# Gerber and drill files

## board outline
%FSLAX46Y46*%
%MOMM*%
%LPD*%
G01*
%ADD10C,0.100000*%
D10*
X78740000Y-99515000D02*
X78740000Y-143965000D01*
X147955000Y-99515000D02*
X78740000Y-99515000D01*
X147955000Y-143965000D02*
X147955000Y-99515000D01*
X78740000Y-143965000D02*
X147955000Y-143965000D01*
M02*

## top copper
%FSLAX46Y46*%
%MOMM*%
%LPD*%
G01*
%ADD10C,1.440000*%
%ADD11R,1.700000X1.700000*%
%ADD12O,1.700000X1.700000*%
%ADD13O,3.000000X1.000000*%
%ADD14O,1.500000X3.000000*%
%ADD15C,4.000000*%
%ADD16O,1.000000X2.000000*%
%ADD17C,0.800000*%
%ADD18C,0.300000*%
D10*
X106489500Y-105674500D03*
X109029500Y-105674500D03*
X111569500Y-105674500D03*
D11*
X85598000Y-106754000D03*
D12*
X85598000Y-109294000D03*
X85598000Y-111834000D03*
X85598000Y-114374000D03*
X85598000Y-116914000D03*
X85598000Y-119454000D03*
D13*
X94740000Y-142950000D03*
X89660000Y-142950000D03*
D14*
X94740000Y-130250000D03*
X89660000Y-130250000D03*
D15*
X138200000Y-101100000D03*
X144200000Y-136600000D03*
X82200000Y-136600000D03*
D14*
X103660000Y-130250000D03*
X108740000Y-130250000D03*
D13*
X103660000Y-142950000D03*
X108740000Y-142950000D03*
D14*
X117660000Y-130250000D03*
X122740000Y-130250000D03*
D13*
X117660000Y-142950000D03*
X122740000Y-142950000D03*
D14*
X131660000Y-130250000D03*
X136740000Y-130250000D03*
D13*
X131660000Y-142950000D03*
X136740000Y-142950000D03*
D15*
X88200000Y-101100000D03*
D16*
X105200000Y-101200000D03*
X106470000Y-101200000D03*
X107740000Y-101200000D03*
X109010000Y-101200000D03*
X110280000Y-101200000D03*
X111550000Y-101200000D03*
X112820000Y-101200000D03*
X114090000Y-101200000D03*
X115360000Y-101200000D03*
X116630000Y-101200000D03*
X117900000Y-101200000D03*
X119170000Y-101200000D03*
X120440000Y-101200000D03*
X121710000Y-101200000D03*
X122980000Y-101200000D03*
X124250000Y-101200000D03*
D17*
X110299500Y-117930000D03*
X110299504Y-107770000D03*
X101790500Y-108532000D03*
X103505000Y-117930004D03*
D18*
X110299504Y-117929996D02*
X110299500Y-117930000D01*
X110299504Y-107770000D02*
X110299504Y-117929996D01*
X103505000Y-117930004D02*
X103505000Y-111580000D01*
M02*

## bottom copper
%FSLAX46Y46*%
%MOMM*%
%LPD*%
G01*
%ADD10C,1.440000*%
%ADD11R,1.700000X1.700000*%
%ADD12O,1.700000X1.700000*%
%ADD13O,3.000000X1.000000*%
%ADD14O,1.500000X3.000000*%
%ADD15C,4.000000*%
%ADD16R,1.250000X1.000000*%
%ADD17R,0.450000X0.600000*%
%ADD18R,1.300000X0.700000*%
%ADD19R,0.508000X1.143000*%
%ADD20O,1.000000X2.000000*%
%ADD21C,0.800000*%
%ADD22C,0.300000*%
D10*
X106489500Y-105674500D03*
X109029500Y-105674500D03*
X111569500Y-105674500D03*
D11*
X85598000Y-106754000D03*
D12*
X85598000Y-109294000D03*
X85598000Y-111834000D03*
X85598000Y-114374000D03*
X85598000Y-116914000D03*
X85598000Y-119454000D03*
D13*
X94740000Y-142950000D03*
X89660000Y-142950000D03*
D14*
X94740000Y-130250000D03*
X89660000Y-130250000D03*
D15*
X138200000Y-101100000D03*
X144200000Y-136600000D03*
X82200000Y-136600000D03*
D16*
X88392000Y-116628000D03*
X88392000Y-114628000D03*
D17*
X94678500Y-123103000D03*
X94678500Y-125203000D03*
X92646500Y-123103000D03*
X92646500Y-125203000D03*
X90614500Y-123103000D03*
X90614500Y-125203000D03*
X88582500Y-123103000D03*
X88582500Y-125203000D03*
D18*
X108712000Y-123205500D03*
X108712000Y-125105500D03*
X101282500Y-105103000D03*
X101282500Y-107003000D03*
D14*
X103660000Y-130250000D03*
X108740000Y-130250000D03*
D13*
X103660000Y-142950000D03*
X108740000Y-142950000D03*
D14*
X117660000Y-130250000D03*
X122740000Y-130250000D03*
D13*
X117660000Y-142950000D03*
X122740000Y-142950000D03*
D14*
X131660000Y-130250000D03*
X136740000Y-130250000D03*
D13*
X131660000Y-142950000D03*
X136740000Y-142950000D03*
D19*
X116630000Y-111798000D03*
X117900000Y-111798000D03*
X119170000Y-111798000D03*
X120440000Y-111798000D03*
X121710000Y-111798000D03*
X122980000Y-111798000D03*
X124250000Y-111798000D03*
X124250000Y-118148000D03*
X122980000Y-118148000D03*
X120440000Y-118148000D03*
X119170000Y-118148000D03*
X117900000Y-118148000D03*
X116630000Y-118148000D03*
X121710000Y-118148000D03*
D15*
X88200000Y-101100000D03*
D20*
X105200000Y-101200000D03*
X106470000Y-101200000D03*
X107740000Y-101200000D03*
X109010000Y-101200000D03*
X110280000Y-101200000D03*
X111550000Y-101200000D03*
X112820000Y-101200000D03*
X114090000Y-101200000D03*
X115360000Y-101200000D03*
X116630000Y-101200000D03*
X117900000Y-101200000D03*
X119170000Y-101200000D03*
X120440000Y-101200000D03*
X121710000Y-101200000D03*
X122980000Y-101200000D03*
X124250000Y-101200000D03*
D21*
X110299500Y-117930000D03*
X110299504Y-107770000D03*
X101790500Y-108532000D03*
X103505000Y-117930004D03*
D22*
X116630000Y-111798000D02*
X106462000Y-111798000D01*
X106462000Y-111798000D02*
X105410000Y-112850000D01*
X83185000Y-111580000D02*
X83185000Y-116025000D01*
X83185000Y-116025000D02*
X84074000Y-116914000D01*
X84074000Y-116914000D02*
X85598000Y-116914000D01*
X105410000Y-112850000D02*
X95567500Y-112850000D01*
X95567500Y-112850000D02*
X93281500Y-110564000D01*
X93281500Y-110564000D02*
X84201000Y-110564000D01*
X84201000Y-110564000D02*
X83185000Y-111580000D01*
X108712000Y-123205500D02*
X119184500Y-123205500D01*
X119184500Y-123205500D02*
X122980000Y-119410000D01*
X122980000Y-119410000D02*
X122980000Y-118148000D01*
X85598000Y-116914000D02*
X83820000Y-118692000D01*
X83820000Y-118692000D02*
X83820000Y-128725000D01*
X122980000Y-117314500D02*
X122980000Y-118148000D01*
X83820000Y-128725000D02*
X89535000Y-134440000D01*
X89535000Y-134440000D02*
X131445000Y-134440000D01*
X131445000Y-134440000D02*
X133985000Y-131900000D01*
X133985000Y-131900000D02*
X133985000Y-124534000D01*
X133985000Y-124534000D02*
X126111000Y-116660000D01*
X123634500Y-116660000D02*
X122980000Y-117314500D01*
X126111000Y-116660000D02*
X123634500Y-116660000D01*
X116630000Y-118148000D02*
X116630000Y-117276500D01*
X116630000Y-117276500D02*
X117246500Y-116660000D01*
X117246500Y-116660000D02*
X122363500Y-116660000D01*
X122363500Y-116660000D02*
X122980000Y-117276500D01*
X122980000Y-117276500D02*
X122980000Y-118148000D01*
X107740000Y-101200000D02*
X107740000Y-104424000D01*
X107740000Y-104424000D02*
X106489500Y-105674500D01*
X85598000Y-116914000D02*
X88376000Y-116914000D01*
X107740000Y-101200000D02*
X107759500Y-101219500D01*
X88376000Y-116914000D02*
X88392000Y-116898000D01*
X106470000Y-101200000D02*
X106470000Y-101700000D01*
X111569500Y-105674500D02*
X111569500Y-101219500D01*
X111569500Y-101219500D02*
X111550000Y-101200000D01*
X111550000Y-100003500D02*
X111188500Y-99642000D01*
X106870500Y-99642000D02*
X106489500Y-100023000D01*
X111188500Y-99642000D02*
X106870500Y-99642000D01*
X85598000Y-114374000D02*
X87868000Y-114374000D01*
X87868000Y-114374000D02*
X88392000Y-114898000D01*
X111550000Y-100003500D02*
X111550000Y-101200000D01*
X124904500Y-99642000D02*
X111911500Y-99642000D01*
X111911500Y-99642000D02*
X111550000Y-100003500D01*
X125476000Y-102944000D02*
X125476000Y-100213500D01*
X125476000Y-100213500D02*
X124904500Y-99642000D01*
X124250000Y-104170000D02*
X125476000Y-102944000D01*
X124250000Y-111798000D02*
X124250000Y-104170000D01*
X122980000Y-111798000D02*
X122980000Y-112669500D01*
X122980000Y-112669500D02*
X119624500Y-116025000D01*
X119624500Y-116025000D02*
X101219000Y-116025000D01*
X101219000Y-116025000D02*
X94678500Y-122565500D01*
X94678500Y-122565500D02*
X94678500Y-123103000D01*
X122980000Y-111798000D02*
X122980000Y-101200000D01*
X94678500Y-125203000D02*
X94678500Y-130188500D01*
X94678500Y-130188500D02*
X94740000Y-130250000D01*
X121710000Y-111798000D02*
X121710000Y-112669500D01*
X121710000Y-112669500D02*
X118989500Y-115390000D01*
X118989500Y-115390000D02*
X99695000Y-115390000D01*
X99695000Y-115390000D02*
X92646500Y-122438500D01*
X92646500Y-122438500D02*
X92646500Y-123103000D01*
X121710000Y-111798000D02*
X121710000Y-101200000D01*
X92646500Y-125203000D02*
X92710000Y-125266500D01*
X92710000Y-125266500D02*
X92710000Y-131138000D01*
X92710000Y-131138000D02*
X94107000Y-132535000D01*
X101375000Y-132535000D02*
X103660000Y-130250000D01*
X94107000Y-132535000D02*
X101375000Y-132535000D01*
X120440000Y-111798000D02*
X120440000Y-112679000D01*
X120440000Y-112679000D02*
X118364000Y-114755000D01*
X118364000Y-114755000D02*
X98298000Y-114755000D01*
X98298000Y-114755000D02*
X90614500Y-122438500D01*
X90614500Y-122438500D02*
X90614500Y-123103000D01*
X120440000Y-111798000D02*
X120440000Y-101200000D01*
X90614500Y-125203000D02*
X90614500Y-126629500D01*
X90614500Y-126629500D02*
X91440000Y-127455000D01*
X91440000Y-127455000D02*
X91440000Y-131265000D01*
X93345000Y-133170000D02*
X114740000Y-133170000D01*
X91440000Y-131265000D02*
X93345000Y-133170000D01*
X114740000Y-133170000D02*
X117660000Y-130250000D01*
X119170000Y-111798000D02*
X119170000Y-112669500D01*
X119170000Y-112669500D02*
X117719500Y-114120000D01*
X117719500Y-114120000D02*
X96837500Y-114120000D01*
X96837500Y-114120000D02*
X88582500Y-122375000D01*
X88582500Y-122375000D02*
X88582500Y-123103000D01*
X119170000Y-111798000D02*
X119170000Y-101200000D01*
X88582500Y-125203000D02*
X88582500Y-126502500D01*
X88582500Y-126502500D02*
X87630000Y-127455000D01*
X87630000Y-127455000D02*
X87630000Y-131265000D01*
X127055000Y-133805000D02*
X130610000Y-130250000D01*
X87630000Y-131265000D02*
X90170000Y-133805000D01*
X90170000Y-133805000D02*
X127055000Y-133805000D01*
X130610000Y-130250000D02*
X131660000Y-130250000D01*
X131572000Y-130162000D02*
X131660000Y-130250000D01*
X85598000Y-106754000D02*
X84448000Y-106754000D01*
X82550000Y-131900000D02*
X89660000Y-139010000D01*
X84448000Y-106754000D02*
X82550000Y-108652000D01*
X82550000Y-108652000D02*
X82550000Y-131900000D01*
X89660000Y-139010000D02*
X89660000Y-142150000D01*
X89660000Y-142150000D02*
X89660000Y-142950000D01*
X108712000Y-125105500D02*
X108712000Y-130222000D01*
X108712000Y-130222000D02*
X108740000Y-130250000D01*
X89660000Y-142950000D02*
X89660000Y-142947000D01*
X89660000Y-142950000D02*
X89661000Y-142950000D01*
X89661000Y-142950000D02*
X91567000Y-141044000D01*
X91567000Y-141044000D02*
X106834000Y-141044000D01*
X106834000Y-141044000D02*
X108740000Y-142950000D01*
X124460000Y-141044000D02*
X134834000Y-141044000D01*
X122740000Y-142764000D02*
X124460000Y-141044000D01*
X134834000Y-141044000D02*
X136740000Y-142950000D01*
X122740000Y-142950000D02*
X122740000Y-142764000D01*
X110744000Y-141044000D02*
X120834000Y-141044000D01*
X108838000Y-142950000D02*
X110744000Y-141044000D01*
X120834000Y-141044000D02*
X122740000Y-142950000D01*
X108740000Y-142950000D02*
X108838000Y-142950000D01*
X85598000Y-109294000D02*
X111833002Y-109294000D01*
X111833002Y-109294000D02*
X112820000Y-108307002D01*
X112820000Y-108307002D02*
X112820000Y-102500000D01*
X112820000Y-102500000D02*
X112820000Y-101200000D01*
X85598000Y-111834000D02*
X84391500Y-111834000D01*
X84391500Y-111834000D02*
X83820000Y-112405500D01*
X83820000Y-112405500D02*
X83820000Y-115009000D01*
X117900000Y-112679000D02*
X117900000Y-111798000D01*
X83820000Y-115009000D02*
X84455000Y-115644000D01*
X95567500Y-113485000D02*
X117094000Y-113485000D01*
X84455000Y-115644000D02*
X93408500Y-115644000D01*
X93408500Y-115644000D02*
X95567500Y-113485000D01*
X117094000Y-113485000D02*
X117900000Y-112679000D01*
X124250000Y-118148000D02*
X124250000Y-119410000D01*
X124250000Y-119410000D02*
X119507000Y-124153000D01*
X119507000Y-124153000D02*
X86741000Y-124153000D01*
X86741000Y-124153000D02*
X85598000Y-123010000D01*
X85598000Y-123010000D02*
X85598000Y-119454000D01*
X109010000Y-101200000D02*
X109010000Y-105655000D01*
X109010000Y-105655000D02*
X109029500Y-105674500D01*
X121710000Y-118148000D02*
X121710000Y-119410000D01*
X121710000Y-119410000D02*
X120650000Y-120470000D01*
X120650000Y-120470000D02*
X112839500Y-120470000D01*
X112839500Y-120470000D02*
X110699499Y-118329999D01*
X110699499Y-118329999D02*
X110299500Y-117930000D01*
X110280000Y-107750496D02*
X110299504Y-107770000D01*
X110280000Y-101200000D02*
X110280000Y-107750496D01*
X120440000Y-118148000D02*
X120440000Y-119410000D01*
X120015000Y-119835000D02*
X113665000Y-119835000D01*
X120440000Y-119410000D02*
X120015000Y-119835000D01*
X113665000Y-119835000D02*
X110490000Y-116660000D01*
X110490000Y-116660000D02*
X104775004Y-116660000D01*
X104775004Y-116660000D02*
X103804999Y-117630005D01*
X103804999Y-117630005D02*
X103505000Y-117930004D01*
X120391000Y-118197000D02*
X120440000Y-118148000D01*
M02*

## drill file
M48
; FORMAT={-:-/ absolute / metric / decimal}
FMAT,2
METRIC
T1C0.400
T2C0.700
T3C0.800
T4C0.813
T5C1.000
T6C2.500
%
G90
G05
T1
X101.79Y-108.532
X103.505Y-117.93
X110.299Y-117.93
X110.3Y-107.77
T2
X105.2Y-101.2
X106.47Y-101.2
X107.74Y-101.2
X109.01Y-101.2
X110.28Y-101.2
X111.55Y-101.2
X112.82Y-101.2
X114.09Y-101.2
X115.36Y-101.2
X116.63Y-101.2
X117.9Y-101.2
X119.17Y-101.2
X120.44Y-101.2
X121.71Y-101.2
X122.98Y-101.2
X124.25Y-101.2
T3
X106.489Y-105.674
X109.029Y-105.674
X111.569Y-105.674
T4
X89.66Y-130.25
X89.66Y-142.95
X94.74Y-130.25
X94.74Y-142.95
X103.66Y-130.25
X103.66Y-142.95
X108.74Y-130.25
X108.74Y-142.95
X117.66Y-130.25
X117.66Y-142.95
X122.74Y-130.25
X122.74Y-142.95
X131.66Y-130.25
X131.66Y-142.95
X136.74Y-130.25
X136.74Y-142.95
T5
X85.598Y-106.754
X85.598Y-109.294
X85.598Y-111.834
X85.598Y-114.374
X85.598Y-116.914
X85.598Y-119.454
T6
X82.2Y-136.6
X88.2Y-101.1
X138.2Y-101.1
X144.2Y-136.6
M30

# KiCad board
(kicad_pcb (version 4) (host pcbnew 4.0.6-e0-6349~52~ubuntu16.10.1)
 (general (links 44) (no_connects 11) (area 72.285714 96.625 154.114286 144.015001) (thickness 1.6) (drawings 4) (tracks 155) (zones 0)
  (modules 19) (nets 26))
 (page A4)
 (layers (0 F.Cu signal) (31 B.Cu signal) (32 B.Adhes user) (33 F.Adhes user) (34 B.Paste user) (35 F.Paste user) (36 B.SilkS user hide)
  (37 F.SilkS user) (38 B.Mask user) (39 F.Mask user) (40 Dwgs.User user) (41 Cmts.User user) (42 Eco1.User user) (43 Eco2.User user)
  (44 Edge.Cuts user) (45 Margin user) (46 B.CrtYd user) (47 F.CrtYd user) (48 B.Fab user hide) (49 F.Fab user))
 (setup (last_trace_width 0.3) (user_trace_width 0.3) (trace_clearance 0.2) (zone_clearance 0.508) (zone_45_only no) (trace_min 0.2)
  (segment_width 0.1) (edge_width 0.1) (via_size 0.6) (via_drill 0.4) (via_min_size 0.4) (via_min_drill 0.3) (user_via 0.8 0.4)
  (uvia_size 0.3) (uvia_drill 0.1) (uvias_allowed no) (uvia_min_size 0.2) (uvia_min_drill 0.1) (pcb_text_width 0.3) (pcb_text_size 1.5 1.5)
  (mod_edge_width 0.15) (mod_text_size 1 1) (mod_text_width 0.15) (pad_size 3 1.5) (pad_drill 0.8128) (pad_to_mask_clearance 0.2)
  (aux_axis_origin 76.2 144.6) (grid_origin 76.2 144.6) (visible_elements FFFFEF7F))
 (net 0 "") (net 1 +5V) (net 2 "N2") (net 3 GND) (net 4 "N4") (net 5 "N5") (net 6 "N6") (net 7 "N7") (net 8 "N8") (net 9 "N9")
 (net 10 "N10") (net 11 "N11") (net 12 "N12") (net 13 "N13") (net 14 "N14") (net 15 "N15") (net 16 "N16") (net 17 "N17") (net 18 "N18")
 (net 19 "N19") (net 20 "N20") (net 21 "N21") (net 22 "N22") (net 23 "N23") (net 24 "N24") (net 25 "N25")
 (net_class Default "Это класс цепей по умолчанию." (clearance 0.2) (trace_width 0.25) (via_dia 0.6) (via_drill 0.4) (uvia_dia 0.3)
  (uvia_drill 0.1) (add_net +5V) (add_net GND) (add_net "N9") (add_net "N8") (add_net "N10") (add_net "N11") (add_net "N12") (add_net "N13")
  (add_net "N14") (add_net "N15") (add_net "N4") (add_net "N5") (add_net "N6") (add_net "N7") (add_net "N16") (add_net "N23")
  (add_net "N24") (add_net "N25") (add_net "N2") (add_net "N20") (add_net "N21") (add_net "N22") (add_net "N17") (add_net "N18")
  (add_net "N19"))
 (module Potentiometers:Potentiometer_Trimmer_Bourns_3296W (layer B.Cu) (at 106.4895 105.6745 180)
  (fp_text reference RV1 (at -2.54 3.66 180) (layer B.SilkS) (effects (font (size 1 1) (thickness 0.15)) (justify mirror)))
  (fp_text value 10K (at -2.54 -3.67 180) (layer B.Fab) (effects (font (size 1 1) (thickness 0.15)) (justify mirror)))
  (pad 1 thru_hole circle (at 0 0 180) (size 1.44 1.44) (drill 0.8) (layers *.Cu *.Mask) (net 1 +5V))
  (pad 2 thru_hole circle (at -2.54 0 180) (size 1.44 1.44) (drill 0.8) (layers *.Cu *.Mask) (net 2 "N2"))
  (pad 3 thru_hole circle (at -5.08 0 180) (size 1.44 1.44) (drill 0.8) (layers *.Cu *.Mask) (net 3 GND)))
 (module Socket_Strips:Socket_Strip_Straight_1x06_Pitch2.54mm (layer B.Cu) (at 85.598 106.754 180)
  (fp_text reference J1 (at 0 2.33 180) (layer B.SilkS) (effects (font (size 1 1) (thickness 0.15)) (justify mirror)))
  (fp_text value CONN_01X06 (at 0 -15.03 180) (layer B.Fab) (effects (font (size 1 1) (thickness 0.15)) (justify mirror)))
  (pad 1 thru_hole rect (at 0 0 180) (size 1.7 1.7) (drill 1) (layers *.Cu *.Mask) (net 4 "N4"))
  (pad 2 thru_hole oval (at 0 -2.54 180) (size 1.7 1.7) (drill 1) (layers *.Cu *.Mask) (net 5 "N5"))
  (pad 3 thru_hole oval (at 0 -5.08 180) (size 1.7 1.7) (drill 1) (layers *.Cu *.Mask) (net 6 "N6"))
  (pad 4 thru_hole oval (at 0 -7.62 180) (size 1.7 1.7) (drill 1) (layers *.Cu *.Mask) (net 3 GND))
  (pad 5 thru_hole oval (at 0 -10.16 180) (size 1.7 1.7) (drill 1) (layers *.Cu *.Mask) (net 1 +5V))
  (pad 6 thru_hole oval (at 0 -12.7 180) (size 1.7 1.7) (drill 1) (layers *.Cu *.Mask) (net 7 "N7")))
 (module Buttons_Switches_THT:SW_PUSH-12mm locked (layer F.Cu) (at 92.2 136.6 270)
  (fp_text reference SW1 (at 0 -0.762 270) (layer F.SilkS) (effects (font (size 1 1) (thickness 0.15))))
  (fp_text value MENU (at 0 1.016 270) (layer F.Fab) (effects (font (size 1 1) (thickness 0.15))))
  (pad 1 thru_hole oval (at 6.35 -2.54) (size 3 1) (drill 0.8128) (layers *.Cu *.Mask) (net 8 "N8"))
  (pad 2 thru_hole oval (at 6.35 2.54) (size 3 1) (drill 0.8128) (layers *.Cu *.Mask) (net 4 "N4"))
  (pad 1 thru_hole oval (at -6.35 -2.54 270) (size 3 1.5) (drill 0.8128) (layers *.Cu *.Mask) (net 8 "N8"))
  (pad 2 thru_hole oval (at -6.35 2.54 270) (size 3 1.5) (drill 0.8128) (layers *.Cu *.Mask) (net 4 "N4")))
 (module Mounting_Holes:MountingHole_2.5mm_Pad (layer F.Cu) (at 138.2 101.1)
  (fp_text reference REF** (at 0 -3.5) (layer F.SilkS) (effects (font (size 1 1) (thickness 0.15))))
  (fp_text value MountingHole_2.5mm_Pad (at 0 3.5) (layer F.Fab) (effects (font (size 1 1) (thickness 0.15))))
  (pad 1 thru_hole circle (at 0 0) (size 4 4) (drill 2.5) (layers *.Cu *.Mask)))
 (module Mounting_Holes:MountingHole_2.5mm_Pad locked (layer F.Cu) (at 144.2 136.6)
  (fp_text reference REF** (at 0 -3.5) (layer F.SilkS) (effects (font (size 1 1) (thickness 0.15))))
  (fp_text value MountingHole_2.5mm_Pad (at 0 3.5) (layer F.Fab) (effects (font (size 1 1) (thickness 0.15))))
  (pad 1 thru_hole circle (at 0 0) (size 4 4) (drill 2.5) (layers *.Cu *.Mask)))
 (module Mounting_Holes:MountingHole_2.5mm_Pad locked (layer F.Cu) (at 82.2 136.6)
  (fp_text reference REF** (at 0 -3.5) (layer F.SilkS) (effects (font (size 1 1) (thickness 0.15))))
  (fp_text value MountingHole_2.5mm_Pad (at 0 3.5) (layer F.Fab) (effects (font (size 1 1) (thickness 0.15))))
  (pad 1 thru_hole circle (at 0 0) (size 4 4) (drill 2.5) (layers *.Cu *.Mask)))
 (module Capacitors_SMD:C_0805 (layer B.Cu) (at 88.392 115.628 90)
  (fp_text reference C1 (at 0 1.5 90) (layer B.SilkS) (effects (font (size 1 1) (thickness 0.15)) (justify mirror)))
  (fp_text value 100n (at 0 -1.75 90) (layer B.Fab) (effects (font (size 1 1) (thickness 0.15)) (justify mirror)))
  (pad 1 smd rect (at -1 0 90) (size 1 1.25) (layers B.Cu B.Paste B.Mask) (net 1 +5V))
  (pad 2 smd rect (at 1 0 90) (size 1 1.25) (layers B.Cu B.Paste B.Mask) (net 3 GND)))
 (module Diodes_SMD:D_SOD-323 (layer B.Cu) (at 94.6785 124.153 270)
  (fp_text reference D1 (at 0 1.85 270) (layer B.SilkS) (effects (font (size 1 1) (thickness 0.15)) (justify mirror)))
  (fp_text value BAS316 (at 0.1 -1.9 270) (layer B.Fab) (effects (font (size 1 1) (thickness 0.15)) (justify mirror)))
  (pad 1 smd rect (at -1.05 0 270) (size 0.6 0.45) (layers B.Cu B.Paste B.Mask) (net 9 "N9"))
  (pad 2 smd rect (at 1.05 0 270) (size 0.6 0.45) (layers B.Cu B.Paste B.Mask) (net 8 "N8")))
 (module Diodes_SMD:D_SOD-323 (layer B.Cu) (at 92.6465 124.153 270)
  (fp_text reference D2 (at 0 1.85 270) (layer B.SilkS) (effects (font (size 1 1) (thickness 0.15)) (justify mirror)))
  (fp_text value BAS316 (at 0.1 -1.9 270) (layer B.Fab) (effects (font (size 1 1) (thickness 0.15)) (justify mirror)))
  (pad 1 smd rect (at -1.05 0 270) (size 0.6 0.45) (layers B.Cu B.Paste B.Mask) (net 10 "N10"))
  (pad 2 smd rect (at 1.05 0 270) (size 0.6 0.45) (layers B.Cu B.Paste B.Mask) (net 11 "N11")))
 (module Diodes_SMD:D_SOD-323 (layer B.Cu) (at 90.6145 124.153 270)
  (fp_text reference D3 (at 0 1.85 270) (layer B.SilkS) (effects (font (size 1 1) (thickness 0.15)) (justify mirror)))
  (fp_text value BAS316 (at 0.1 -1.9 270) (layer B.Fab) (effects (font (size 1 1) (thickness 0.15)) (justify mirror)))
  (pad 1 smd rect (at -1.05 0 270) (size 0.6 0.45) (layers B.Cu B.Paste B.Mask) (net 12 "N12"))
  (pad 2 smd rect (at 1.05 0 270) (size 0.6 0.45) (layers B.Cu B.Paste B.Mask) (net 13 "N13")))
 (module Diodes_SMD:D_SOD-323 (layer B.Cu) (at 88.5825 124.153 270)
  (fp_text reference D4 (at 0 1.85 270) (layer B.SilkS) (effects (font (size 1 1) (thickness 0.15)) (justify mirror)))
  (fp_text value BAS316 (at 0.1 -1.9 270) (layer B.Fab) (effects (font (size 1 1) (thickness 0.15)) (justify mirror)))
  (pad 1 smd rect (at -1.05 0 270) (size 0.6 0.45) (layers B.Cu B.Paste B.Mask) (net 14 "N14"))
  (pad 2 smd rect (at 1.05 0 270) (size 0.6 0.45) (layers B.Cu B.Paste B.Mask) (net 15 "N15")))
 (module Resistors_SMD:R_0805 (layer B.Cu) (at 108.712 124.1555 270)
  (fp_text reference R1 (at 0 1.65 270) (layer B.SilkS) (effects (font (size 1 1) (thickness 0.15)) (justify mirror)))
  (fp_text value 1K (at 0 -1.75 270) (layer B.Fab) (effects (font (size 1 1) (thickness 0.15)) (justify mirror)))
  (pad 1 smd rect (at -0.95 0 270) (size 0.7 1.3) (layers B.Cu B.Paste B.Mask) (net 1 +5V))
  (pad 2 smd rect (at 0.95 0 270) (size 0.7 1.3) (layers B.Cu B.Paste B.Mask) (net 4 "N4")))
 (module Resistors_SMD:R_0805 (layer B.Cu) (at 101.2825 106.053 270)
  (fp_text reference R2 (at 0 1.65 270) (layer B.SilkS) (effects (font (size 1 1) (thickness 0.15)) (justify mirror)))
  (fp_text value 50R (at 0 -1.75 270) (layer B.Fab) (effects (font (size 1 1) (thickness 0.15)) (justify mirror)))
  (pad 1 smd rect (at -0.95 0 270) (size 0.7 1.3) (layers B.Cu B.Paste B.Mask) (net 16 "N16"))
  (pad 2 smd rect (at 0.95 0 270) (size 0.7 1.3) (layers B.Cu B.Paste B.Mask) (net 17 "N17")))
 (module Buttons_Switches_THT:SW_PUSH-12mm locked (layer F.Cu) (at 106.2 136.6 90)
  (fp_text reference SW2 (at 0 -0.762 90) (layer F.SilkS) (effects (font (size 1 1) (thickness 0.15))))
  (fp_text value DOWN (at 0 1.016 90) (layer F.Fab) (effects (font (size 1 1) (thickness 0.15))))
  (pad 1 thru_hole oval (at 6.35 -2.54 90) (size 3 1.5) (drill 0.8128) (layers *.Cu *.Mask) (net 11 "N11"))
  (pad 2 thru_hole oval (at 6.35 2.54 90) (size 3 1.5) (drill 0.8128) (layers *.Cu *.Mask) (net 4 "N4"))
  (pad 1 thru_hole oval (at -6.35 -2.54 180) (size 3 1) (drill 0.8128) (layers *.Cu *.Mask) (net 11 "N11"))
  (pad 2 thru_hole oval (at -6.35 2.54 180) (size 3 1) (drill 0.8128) (layers *.Cu *.Mask) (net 4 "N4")))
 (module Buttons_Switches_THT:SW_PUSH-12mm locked (layer F.Cu) (at 120.2 136.6 90)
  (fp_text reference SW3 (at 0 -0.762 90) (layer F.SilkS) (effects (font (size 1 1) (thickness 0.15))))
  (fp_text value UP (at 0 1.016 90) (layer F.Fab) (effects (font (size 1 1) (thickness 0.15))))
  (pad 1 thru_hole oval (at 6.35 -2.54 90) (size 3 1.5) (drill 0.8128) (layers *.Cu *.Mask) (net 13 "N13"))
  (pad 2 thru_hole oval (at 6.35 2.54 90) (size 3 1.5) (drill 0.8128) (layers *.Cu *.Mask) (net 4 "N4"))
  (pad 1 thru_hole oval (at -6.35 -2.54 180) (size 3 1) (drill 0.8128) (layers *.Cu *.Mask) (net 13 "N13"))
  (pad 2 thru_hole oval (at -6.35 2.54 180) (size 3 1) (drill 0.8128) (layers *.Cu *.Mask) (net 4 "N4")))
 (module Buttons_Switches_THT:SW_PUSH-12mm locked (layer F.Cu) (at 134.2 136.6 90)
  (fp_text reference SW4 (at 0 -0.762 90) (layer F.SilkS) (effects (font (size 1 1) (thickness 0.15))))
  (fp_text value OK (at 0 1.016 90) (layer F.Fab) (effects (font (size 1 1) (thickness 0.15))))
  (pad 1 thru_hole oval (at 6.35 -2.54 90) (size 3 1.5) (drill 0.8128) (layers *.Cu *.Mask) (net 15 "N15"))
  (pad 2 thru_hole oval (at 6.35 2.54 90) (size 3 1.5) (drill 0.8128) (layers *.Cu *.Mask) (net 4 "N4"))
  (pad 1 thru_hole oval (at -6.35 -2.54 180) (size 3 1) (drill 0.8128) (layers *.Cu *.Mask) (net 15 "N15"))
  (pad 2 thru_hole oval (at -6.35 2.54 180) (size 3 1) (drill 0.8128) (layers *.Cu *.Mask) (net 4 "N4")))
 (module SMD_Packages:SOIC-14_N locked (layer B.Cu) (at 120.44 115.1)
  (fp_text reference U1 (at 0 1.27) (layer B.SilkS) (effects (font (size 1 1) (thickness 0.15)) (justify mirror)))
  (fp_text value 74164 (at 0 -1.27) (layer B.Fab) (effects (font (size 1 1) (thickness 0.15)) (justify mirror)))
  (pad 1 smd rect (at -3.81 -3.302) (size 0.508 1.143) (layers B.Cu B.Paste B.Mask) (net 1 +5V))
  (pad 2 smd rect (at -2.54 -3.302) (size 0.508 1.143) (layers B.Cu B.Paste B.Mask) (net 6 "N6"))
  (pad 3 smd rect (at -1.27 -3.302) (size 0.508 1.143) (layers B.Cu B.Paste B.Mask) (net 14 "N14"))
  (pad 4 smd rect (at 0 -3.302) (size 0.508 1.143) (layers B.Cu B.Paste B.Mask) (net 12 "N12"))
  (pad 5 smd rect (at 1.27 -3.302) (size 0.508 1.143) (layers B.Cu B.Paste B.Mask) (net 10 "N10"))
  (pad 6 smd rect (at 2.54 -3.302) (size 0.508 1.143) (layers B.Cu B.Paste B.Mask) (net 9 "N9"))
  (pad 7 smd rect (at 3.81 -3.302) (size 0.508 1.143) (layers B.Cu B.Paste B.Mask) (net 3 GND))
  (pad 8 smd rect (at 3.81 3.048) (size 0.508 1.143) (layers B.Cu B.Paste B.Mask) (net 7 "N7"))
  (pad 9 smd rect (at 2.54 3.048) (size 0.508 1.143) (layers B.Cu B.Paste B.Mask) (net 1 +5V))
  (pad 11 smd rect (at 0 3.048) (size 0.508 1.143) (layers B.Cu B.Paste B.Mask) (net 17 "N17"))
  (pad 12 smd rect (at -1.27 3.048) (size 0.508 1.143) (layers B.Cu B.Paste B.Mask) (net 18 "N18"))
  (pad 13 smd rect (at -2.54 3.048) (size 0.508 1.143) (layers B.Cu B.Paste B.Mask) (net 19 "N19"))
  (pad 14 smd rect (at -3.81 3.048) (size 0.508 1.143) (layers B.Cu B.Paste B.Mask) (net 1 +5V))
  (pad 10 smd rect (at 1.27 3.048) (size 0.508 1.143) (layers B.Cu B.Paste B.Mask) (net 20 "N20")))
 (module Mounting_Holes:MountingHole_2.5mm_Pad (layer F.Cu) (at 88.2 101.1)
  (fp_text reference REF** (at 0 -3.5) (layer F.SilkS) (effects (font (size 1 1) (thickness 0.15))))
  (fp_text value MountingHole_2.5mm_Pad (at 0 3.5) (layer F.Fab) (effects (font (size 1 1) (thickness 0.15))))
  (pad 1 thru_hole circle (at 0 0) (size 4 4) (drill 2.5) (layers *.Cu *.Mask)))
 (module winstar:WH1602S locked (layer F.Cu) (at 113.2 115.1)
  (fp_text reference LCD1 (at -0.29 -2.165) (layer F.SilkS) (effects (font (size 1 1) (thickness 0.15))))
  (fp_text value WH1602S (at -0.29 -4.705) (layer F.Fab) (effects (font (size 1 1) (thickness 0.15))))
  (pad 1 thru_hole oval (at -8 -13.9) (size 1 2) (drill 0.7) (layers *.Cu *.Mask) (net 16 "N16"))
  (pad 2 thru_hole oval (at -6.73 -13.9) (size 1 2) (drill 0.7) (layers *.Cu *.Mask) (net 3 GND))
  (pad 3 thru_hole oval (at -5.46 -13.9) (size 1 2) (drill 0.7) (layers *.Cu *.Mask) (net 1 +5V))
  (pad 4 thru_hole oval (at -4.19 -13.9) (size 1 2) (drill 0.7) (layers *.Cu *.Mask) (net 2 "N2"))
  (pad 5 thru_hole oval (at -2.92 -13.9) (size 1 2) (drill 0.7) (layers *.Cu *.Mask) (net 20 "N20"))
  (pad 6 thru_hole oval (at -1.65 -13.9) (size 1 2) (drill 0.7) (layers *.Cu *.Mask) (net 3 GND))
  (pad 7 thru_hole oval (at -0.38 -13.9) (size 1 2) (drill 0.7) (layers *.Cu *.Mask) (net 5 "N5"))
  (pad 8 thru_hole oval (at 0.89 -13.9) (size 1 2) (drill 0.7) (layers *.Cu *.Mask) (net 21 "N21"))
  (pad 9 thru_hole oval (at 2.16 -13.9) (size 1 2) (drill 0.7) (layers *.Cu *.Mask) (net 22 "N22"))
  (pad 10 thru_hole oval (at 3.43 -13.9) (size 1 2) (drill 0.7) (layers *.Cu *.Mask) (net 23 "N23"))
  (pad 11 thru_hole oval (at 4.7 -13.9) (size 1 2) (drill 0.7) (layers *.Cu *.Mask) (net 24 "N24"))
  (pad 12 thru_hole oval (at 5.97 -13.9) (size 1 2) (drill 0.7) (layers *.Cu *.Mask) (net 14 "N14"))
  (pad 13 thru_hole oval (at 7.24 -13.9) (size 1 2) (drill 0.7) (layers *.Cu *.Mask) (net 12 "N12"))
  (pad 14 thru_hole oval (at 8.51 -13.9) (size 1 2) (drill 0.7) (layers *.Cu *.Mask) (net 10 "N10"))
  (pad 15 thru_hole oval (at 9.78 -13.9) (size 1 2) (drill 0.7) (layers *.Cu *.Mask) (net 9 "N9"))
  (pad 16 thru_hole oval (at 11.05 -13.9) (size 1 2) (drill 0.7) (layers *.Cu *.Mask) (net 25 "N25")))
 (gr_line (start 78.74 99.515) (end 78.74 143.965) (layer Edge.Cuts) (width 0.1))
 (gr_line (start 147.955 99.515) (end 78.74 99.515) (layer Edge.Cuts) (width 0.1))
 (gr_line (start 147.955 143.965) (end 147.955 99.515) (layer Edge.Cuts) (width 0.1))
 (gr_line (start 78.74 143.965) (end 147.955 143.965) (layer Edge.Cuts) (width 0.1))
 (segment (start 116.63 111.798) (end 106.462 111.798) (width 0.3) (layer B.Cu) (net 1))
 (segment (start 106.462 111.798) (end 105.41 112.85) (width 0.3) (layer B.Cu) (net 1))
 (segment (start 83.185 111.58) (end 83.185 116.025) (width 0.3) (layer B.Cu) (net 1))
 (segment (start 83.185 116.025) (end 84.074 116.914) (width 0.3) (layer B.Cu) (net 1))
 (segment (start 84.074 116.914) (end 85.598 116.914) (width 0.3) (layer B.Cu) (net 1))
 (segment (start 105.41 112.85) (end 95.5675 112.85) (width 0.3) (layer B.Cu) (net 1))
 (segment (start 95.5675 112.85) (end 93.2815 110.564) (width 0.3) (layer B.Cu) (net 1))
 (segment (start 93.2815 110.564) (end 84.201 110.564) (width 0.3) (layer B.Cu) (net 1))
 (segment (start 84.201 110.564) (end 83.185 111.58) (width 0.3) (layer B.Cu) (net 1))
 (segment (start 108.712 123.2055) (end 119.1845 123.2055) (width 0.3) (layer B.Cu) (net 1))
 (segment (start 119.1845 123.2055) (end 122.98 119.41) (width 0.3) (layer B.Cu) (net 1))
 (segment (start 122.98 119.41) (end 122.98 118.148) (width 0.3) (layer B.Cu) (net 1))
 (segment (start 85.598 116.914) (end 83.82 118.692) (width 0.3) (layer B.Cu) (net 1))
 (segment (start 83.82 118.692) (end 83.82 128.725) (width 0.3) (layer B.Cu) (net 1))
 (segment (start 122.98 117.3145) (end 122.98 118.148) (width 0.3) (layer B.Cu) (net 1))
 (segment (start 83.82 128.725) (end 89.535 134.44) (width 0.3) (layer B.Cu) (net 1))
 (segment (start 89.535 134.44) (end 131.445 134.44) (width 0.3) (layer B.Cu) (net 1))
 (segment (start 131.445 134.44) (end 133.985 131.9) (width 0.3) (layer B.Cu) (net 1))
 (segment (start 133.985 131.9) (end 133.985 124.534) (width 0.3) (layer B.Cu) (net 1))
 (segment (start 133.985 124.534) (end 126.111 116.66) (width 0.3) (layer B.Cu) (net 1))
 (segment (start 123.6345 116.66) (end 122.98 117.3145) (width 0.3) (layer B.Cu) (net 1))
 (segment (start 126.111 116.66) (end 123.6345 116.66) (width 0.3) (layer B.Cu) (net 1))
 (segment (start 116.63 118.148) (end 116.63 117.2765) (width 0.3) (layer B.Cu) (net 1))
 (segment (start 116.63 117.2765) (end 117.2465 116.66) (width 0.3) (layer B.Cu) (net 1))
 (segment (start 117.2465 116.66) (end 122.3635 116.66) (width 0.3) (layer B.Cu) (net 1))
 (segment (start 122.3635 116.66) (end 122.98 117.2765) (width 0.3) (layer B.Cu) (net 1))
 (segment (start 122.98 117.2765) (end 122.98 118.148) (width 0.3) (layer B.Cu) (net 1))
 (segment (start 107.74 101.2) (end 107.74 104.424) (width 0.3) (layer B.Cu) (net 1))
 (segment (start 107.74 104.424) (end 106.4895 105.6745) (width 0.3) (layer B.Cu) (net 1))
 (segment (start 85.598 116.914) (end 88.376 116.914) (width 0.3) (layer B.Cu) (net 1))
 (segment (start 107.74 101.2) (end 107.7595 101.2195) (width 0.3) (layer B.Cu) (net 1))
 (segment (start 88.376 116.914) (end 88.392 116.898) (width 0.3) (layer B.Cu) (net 1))
 (segment (start 106.47 101.2) (end 106.47 101.7) (width 0.3) (layer B.Cu) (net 3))
 (segment (start 111.5695 105.6745) (end 111.5695 101.2195) (width 0.3) (layer B.Cu) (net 3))
 (segment (start 111.5695 101.2195) (end 111.55 101.2) (width 0.3) (layer B.Cu) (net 3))
 (segment (start 111.55 100.0035) (end 111.1885 99.642) (width 0.3) (layer B.Cu) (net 3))
 (segment (start 106.8705 99.642) (end 106.4895 100.023) (width 0.3) (layer B.Cu) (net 3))
 (segment (start 111.1885 99.642) (end 106.8705 99.642) (width 0.3) (layer B.Cu) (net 3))
 (segment (start 85.598 114.374) (end 87.868 114.374) (width 0.3) (layer B.Cu) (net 3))
 (segment (start 87.868 114.374) (end 88.392 114.898) (width 0.3) (layer B.Cu) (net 3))
 (segment (start 111.55 100.0035) (end 111.55 101.2) (width 0.3) (layer B.Cu) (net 3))
 (segment (start 124.9045 99.642) (end 111.9115 99.642) (width 0.3) (layer B.Cu) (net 3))
 (segment (start 111.9115 99.642) (end 111.55 100.0035) (width 0.3) (layer B.Cu) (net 3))
 (segment (start 125.476 102.944) (end 125.476 100.2135) (width 0.3) (layer B.Cu) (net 3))
 (segment (start 125.476 100.2135) (end 124.9045 99.642) (width 0.3) (layer B.Cu) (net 3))
 (segment (start 124.25 104.17) (end 125.476 102.944) (width 0.3) (layer B.Cu) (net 3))
 (segment (start 124.25 111.798) (end 124.25 104.17) (width 0.3) (layer B.Cu) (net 3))
 (segment (start 122.98 111.798) (end 122.98 112.6695) (width 0.3) (layer B.Cu) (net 9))
 (segment (start 122.98 112.6695) (end 119.6245 116.025) (width 0.3) (layer B.Cu) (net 9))
 (segment (start 119.6245 116.025) (end 101.219 116.025) (width 0.3) (layer B.Cu) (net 9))
 (segment (start 101.219 116.025) (end 94.6785 122.5655) (width 0.3) (layer B.Cu) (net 9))
 (segment (start 94.6785 122.5655) (end 94.6785 123.103) (width 0.3) (layer B.Cu) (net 9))
 (segment (start 122.98 111.798) (end 122.98 101.2) (width 0.3) (layer B.Cu) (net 9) (status 10))
 (segment (start 94.6785 125.203) (end 94.6785 130.1885) (width 0.3) (layer B.Cu) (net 8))
 (segment (start 94.6785 130.1885) (end 94.74 130.25) (width 0.3) (layer B.Cu) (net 8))
 (segment (start 121.71 111.798) (end 121.71 112.6695) (width 0.3) (layer B.Cu) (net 10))
 (segment (start 121.71 112.6695) (end 118.9895 115.39) (width 0.3) (layer B.Cu) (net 10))
 (segment (start 118.9895 115.39) (end 99.695 115.39) (width 0.3) (layer B.Cu) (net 10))
 (segment (start 99.695 115.39) (end 92.6465 122.4385) (width 0.3) (layer B.Cu) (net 10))
 (segment (start 92.6465 122.4385) (end 92.6465 123.103) (width 0.3) (layer B.Cu) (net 10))
 (segment (start 121.71 111.798) (end 121.71 101.2) (width 0.3) (layer B.Cu) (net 10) (status 10))
 (segment (start 92.6465 125.203) (end 92.71 125.2665) (width 0.3) (layer B.Cu) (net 11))
 (segment (start 92.71 125.2665) (end 92.71 131.138) (width 0.3) (layer B.Cu) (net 11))
 (segment (start 92.71 131.138) (end 94.107 132.535) (width 0.3) (layer B.Cu) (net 11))
 (segment (start 101.375 132.535) (end 103.66 130.25) (width 0.3) (layer B.Cu) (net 11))
 (segment (start 94.107 132.535) (end 101.375 132.535) (width 0.3) (layer B.Cu) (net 11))
 (segment (start 120.44 111.798) (end 120.44 112.679) (width 0.3) (layer B.Cu) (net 12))
 (segment (start 120.44 112.679) (end 118.364 114.755) (width 0.3) (layer B.Cu) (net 12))
 (segment (start 118.364 114.755) (end 98.298 114.755) (width 0.3) (layer B.Cu) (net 12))
 (segment (start 98.298 114.755) (end 90.6145 122.4385) (width 0.3) (layer B.Cu) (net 12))
 (segment (start 90.6145 122.4385) (end 90.6145 123.103) (width 0.3) (layer B.Cu) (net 12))
 (segment (start 120.44 111.798) (end 120.44 101.2) (width 0.3) (layer B.Cu) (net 12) (status 10))
 (segment (start 90.6145 125.203) (end 90.6145 126.6295) (width 0.3) (layer B.Cu) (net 13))
 (segment (start 90.6145 126.6295) (end 91.44 127.455) (width 0.3) (layer B.Cu) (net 13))
 (segment (start 91.44 127.455) (end 91.44 131.265) (width 0.3) (layer B.Cu) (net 13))
 (segment (start 93.345 133.17) (end 114.74 133.17) (width 0.3) (layer B.Cu) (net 13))
 (segment (start 91.44 131.265) (end 93.345 133.17) (width 0.3) (layer B.Cu) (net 13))
 (segment (start 114.74 133.17) (end 117.66 130.25) (width 0.3) (layer B.Cu) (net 13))
 (segment (start 119.17 111.798) (end 119.17 112.6695) (width 0.3) (layer B.Cu) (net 14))
 (segment (start 119.17 112.6695) (end 117.7195 114.12) (width 0.3) (layer B.Cu) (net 14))
 (segment (start 117.7195 114.12) (end 96.8375 114.12) (width 0.3) (layer B.Cu) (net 14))
 (segment (start 96.8375 114.12) (end 88.5825 122.375) (width 0.3) (layer B.Cu) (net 14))
 (segment (start 88.5825 122.375) (end 88.5825 123.103) (width 0.3) (layer B.Cu) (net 14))
 (segment (start 119.17 111.798) (end 119.17 101.2) (width 0.3) (layer B.Cu) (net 14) (status 10))
 (segment (start 88.5825 125.203) (end 88.5825 126.5025) (width 0.3) (layer B.Cu) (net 15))
 (segment (start 88.5825 126.5025) (end 87.63 127.455) (width 0.3) (layer B.Cu) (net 15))
 (segment (start 87.63 127.455) (end 87.63 131.265) (width 0.3) (layer B.Cu) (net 15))
 (segment (start 127.055 133.805) (end 130.61 130.25) (width 0.3) (layer B.Cu) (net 15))
 (segment (start 87.63 131.265) (end 90.17 133.805) (width 0.3) (layer B.Cu) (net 15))
 (segment (start 90.17 133.805) (end 127.055 133.805) (width 0.3) (layer B.Cu) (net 15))
 (segment (start 130.61 130.25) (end 131.66 130.25) (width 0.3) (layer B.Cu) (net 15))
 (segment (start 131.572 130.162) (end 131.66 130.25) (width 0.3) (layer B.Cu) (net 15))
 (segment (start 85.598 106.754) (end 84.448 106.754) (width 0.3) (layer B.Cu) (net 4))
 (segment (start 82.55 131.9) (end 89.66 139.01) (width 0.3) (layer B.Cu) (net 4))
 (segment (start 84.448 106.754) (end 82.55 108.652) (width 0.3) (layer B.Cu) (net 4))
 (segment (start 82.55 108.652) (end 82.55 131.9) (width 0.3) (layer B.Cu) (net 4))
 (segment (start 89.66 139.01) (end 89.66 142.15) (width 0.3) (layer B.Cu) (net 4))
 (segment (start 89.66 142.15) (end 89.66 142.95) (width 0.3) (layer B.Cu) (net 4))
 (segment (start 108.712 125.1055) (end 108.712 130.222) (width 0.3) (layer B.Cu) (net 4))
 (segment (start 108.712 130.222) (end 108.74 130.25) (width 0.3) (layer B.Cu) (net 4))
 (segment (start 89.66 142.95) (end 89.66 142.947) (width 0.3) (layer B.Cu) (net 4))
 (segment (start 89.66 142.95) (end 89.661 142.95) (width 0.3) (layer B.Cu) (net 4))
 (segment (start 89.661 142.95) (end 91.567 141.044) (width 0.3) (layer B.Cu) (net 4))
 (segment (start 91.567 141.044) (end 106.834 141.044) (width 0.3) (layer B.Cu) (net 4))
 (segment (start 106.834 141.044) (end 108.74 142.95) (width 0.3) (layer B.Cu) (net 4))
 (segment (start 124.46 141.044) (end 134.834 141.044) (width 0.3) (layer B.Cu) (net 4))
 (segment (start 122.74 142.764) (end 124.46 141.044) (width 0.3) (layer B.Cu) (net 4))
 (segment (start 134.834 141.044) (end 136.74 142.95) (width 0.3) (layer B.Cu) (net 4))
 (segment (start 122.74 142.95) (end 122.74 142.764) (width 0.3) (layer B.Cu) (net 4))
 (segment (start 110.744 141.044) (end 120.834 141.044) (width 0.3) (layer B.Cu) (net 4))
 (segment (start 108.838 142.95) (end 110.744 141.044) (width 0.3) (layer B.Cu) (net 4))
 (segment (start 120.834 141.044) (end 122.74 142.95) (width 0.3) (layer B.Cu) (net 4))
 (segment (start 108.74 142.95) (end 108.838 142.95) (width 0.3) (layer B.Cu) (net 4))
 (segment (start 85.598 109.294) (end 111.833002 109.294) (width 0.3) (layer B.Cu) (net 5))
 (segment (start 111.833002 109.294) (end 112.82 108.307002) (width 0.3) (layer B.Cu) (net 5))
 (segment (start 112.82 108.307002) (end 112.82 102.5) (width 0.3) (layer B.Cu) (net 5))
 (segment (start 112.82 102.5) (end 112.82 101.2) (width 0.3) (layer B.Cu) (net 5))
 (segment (start 85.598 111.834) (end 84.3915 111.834) (width 0.3) (layer B.Cu) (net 6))
 (segment (start 84.3915 111.834) (end 83.82 112.4055) (width 0.3) (layer B.Cu) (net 6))
 (segment (start 83.82 112.4055) (end 83.82 115.009) (width 0.3) (layer B.Cu) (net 6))
 (segment (start 117.9 112.679) (end 117.9 111.798) (width 0.3) (layer B.Cu) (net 6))
 (segment (start 83.82 115.009) (end 84.455 115.644) (width 0.3) (layer B.Cu) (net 6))
 (segment (start 95.5675 113.485) (end 117.094 113.485) (width 0.3) (layer B.Cu) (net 6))
 (segment (start 84.455 115.644) (end 93.4085 115.644) (width 0.3) (layer B.Cu) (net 6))
 (segment (start 93.4085 115.644) (end 95.5675 113.485) (width 0.3) (layer B.Cu) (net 6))
 (segment (start 117.094 113.485) (end 117.9 112.679) (width 0.3) (layer B.Cu) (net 6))
 (segment (start 124.25 118.148) (end 124.25 119.41) (width 0.3) (layer B.Cu) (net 7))
 (segment (start 124.25 119.41) (end 119.507 124.153) (width 0.3) (layer B.Cu) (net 7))
 (segment (start 119.507 124.153) (end 86.741 124.153) (width 0.3) (layer B.Cu) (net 7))
 (segment (start 86.741 124.153) (end 85.598 123.01) (width 0.3) (layer B.Cu) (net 7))
 (segment (start 85.598 123.01) (end 85.598 119.454) (width 0.3) (layer B.Cu) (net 7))
 (segment (start 109.01 101.2) (end 109.01 105.655) (width 0.3) (layer B.Cu) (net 2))
 (segment (start 109.01 105.655) (end 109.0295 105.6745) (width 0.3) (layer B.Cu) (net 2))
 (segment (start 121.71 118.148) (end 121.71 119.41) (width 0.3) (layer B.Cu) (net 20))
 (segment (start 121.71 119.41) (end 120.65 120.47) (width 0.3) (layer B.Cu) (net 20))
 (segment (start 120.65 120.47) (end 112.8395 120.47) (width 0.3) (layer B.Cu) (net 20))
 (segment (start 112.8395 120.47) (end 110.699499 118.329999) (width 0.3) (layer B.Cu) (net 20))
 (segment (start 110.699499 118.329999) (end 110.2995 117.93) (width 0.3) (layer B.Cu) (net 20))
 (segment (start 110.299504 117.929996) (end 110.2995 117.93) (width 0.3) (layer F.Cu) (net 20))
 (segment (start 110.299504 107.77) (end 110.299504 117.929996) (width 0.3) (layer F.Cu) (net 20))
 (via (at 110.2995 117.93) (size 0.8) (drill 0.4) (layers F.Cu B.Cu) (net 20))
 (segment (start 110.28 107.750496) (end 110.299504 107.77) (width 0.3) (layer B.Cu) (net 20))
 (segment (start 110.28 101.2) (end 110.28 107.750496) (width 0.3) (layer B.Cu) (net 20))
 (via (at 110.299504 107.77) (size 0.8) (drill 0.4) (layers F.Cu B.Cu) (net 20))
 (segment (start 120.44 118.148) (end 120.44 119.41) (width 0.3) (layer B.Cu) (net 17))
 (segment (start 120.015 119.835) (end 113.665 119.835) (width 0.3) (layer B.Cu) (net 17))
 (segment (start 120.44 119.41) (end 120.015 119.835) (width 0.3) (layer B.Cu) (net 17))
 (segment (start 113.665 119.835) (end 110.49 116.66) (width 0.3) (layer B.Cu) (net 17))
 (segment (start 110.49 116.66) (end 104.775004 116.66) (width 0.3) (layer B.Cu) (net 17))
 (segment (start 104.775004 116.66) (end 103.804999 117.630005) (width 0.3) (layer B.Cu) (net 17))
 (segment (start 103.804999 117.630005) (end 103.505 117.930004) (width 0.3) (layer B.Cu) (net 17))
 (segment (start 103.505 117.930004) (end 103.505 111.58) (width 0.3) (layer F.Cu) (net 17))
 (via (at 101.7905 108.532) (size 0.8) (drill 0.4) (layers F.Cu B.Cu) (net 17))
 (via (at 103.505 117.930004) (size 0.8) (drill 0.4) (layers F.Cu B.Cu) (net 17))
 (segment (start 120.391 118.197) (end 120.44 118.148) (width 0.3) (layer B.Cu) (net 17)))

